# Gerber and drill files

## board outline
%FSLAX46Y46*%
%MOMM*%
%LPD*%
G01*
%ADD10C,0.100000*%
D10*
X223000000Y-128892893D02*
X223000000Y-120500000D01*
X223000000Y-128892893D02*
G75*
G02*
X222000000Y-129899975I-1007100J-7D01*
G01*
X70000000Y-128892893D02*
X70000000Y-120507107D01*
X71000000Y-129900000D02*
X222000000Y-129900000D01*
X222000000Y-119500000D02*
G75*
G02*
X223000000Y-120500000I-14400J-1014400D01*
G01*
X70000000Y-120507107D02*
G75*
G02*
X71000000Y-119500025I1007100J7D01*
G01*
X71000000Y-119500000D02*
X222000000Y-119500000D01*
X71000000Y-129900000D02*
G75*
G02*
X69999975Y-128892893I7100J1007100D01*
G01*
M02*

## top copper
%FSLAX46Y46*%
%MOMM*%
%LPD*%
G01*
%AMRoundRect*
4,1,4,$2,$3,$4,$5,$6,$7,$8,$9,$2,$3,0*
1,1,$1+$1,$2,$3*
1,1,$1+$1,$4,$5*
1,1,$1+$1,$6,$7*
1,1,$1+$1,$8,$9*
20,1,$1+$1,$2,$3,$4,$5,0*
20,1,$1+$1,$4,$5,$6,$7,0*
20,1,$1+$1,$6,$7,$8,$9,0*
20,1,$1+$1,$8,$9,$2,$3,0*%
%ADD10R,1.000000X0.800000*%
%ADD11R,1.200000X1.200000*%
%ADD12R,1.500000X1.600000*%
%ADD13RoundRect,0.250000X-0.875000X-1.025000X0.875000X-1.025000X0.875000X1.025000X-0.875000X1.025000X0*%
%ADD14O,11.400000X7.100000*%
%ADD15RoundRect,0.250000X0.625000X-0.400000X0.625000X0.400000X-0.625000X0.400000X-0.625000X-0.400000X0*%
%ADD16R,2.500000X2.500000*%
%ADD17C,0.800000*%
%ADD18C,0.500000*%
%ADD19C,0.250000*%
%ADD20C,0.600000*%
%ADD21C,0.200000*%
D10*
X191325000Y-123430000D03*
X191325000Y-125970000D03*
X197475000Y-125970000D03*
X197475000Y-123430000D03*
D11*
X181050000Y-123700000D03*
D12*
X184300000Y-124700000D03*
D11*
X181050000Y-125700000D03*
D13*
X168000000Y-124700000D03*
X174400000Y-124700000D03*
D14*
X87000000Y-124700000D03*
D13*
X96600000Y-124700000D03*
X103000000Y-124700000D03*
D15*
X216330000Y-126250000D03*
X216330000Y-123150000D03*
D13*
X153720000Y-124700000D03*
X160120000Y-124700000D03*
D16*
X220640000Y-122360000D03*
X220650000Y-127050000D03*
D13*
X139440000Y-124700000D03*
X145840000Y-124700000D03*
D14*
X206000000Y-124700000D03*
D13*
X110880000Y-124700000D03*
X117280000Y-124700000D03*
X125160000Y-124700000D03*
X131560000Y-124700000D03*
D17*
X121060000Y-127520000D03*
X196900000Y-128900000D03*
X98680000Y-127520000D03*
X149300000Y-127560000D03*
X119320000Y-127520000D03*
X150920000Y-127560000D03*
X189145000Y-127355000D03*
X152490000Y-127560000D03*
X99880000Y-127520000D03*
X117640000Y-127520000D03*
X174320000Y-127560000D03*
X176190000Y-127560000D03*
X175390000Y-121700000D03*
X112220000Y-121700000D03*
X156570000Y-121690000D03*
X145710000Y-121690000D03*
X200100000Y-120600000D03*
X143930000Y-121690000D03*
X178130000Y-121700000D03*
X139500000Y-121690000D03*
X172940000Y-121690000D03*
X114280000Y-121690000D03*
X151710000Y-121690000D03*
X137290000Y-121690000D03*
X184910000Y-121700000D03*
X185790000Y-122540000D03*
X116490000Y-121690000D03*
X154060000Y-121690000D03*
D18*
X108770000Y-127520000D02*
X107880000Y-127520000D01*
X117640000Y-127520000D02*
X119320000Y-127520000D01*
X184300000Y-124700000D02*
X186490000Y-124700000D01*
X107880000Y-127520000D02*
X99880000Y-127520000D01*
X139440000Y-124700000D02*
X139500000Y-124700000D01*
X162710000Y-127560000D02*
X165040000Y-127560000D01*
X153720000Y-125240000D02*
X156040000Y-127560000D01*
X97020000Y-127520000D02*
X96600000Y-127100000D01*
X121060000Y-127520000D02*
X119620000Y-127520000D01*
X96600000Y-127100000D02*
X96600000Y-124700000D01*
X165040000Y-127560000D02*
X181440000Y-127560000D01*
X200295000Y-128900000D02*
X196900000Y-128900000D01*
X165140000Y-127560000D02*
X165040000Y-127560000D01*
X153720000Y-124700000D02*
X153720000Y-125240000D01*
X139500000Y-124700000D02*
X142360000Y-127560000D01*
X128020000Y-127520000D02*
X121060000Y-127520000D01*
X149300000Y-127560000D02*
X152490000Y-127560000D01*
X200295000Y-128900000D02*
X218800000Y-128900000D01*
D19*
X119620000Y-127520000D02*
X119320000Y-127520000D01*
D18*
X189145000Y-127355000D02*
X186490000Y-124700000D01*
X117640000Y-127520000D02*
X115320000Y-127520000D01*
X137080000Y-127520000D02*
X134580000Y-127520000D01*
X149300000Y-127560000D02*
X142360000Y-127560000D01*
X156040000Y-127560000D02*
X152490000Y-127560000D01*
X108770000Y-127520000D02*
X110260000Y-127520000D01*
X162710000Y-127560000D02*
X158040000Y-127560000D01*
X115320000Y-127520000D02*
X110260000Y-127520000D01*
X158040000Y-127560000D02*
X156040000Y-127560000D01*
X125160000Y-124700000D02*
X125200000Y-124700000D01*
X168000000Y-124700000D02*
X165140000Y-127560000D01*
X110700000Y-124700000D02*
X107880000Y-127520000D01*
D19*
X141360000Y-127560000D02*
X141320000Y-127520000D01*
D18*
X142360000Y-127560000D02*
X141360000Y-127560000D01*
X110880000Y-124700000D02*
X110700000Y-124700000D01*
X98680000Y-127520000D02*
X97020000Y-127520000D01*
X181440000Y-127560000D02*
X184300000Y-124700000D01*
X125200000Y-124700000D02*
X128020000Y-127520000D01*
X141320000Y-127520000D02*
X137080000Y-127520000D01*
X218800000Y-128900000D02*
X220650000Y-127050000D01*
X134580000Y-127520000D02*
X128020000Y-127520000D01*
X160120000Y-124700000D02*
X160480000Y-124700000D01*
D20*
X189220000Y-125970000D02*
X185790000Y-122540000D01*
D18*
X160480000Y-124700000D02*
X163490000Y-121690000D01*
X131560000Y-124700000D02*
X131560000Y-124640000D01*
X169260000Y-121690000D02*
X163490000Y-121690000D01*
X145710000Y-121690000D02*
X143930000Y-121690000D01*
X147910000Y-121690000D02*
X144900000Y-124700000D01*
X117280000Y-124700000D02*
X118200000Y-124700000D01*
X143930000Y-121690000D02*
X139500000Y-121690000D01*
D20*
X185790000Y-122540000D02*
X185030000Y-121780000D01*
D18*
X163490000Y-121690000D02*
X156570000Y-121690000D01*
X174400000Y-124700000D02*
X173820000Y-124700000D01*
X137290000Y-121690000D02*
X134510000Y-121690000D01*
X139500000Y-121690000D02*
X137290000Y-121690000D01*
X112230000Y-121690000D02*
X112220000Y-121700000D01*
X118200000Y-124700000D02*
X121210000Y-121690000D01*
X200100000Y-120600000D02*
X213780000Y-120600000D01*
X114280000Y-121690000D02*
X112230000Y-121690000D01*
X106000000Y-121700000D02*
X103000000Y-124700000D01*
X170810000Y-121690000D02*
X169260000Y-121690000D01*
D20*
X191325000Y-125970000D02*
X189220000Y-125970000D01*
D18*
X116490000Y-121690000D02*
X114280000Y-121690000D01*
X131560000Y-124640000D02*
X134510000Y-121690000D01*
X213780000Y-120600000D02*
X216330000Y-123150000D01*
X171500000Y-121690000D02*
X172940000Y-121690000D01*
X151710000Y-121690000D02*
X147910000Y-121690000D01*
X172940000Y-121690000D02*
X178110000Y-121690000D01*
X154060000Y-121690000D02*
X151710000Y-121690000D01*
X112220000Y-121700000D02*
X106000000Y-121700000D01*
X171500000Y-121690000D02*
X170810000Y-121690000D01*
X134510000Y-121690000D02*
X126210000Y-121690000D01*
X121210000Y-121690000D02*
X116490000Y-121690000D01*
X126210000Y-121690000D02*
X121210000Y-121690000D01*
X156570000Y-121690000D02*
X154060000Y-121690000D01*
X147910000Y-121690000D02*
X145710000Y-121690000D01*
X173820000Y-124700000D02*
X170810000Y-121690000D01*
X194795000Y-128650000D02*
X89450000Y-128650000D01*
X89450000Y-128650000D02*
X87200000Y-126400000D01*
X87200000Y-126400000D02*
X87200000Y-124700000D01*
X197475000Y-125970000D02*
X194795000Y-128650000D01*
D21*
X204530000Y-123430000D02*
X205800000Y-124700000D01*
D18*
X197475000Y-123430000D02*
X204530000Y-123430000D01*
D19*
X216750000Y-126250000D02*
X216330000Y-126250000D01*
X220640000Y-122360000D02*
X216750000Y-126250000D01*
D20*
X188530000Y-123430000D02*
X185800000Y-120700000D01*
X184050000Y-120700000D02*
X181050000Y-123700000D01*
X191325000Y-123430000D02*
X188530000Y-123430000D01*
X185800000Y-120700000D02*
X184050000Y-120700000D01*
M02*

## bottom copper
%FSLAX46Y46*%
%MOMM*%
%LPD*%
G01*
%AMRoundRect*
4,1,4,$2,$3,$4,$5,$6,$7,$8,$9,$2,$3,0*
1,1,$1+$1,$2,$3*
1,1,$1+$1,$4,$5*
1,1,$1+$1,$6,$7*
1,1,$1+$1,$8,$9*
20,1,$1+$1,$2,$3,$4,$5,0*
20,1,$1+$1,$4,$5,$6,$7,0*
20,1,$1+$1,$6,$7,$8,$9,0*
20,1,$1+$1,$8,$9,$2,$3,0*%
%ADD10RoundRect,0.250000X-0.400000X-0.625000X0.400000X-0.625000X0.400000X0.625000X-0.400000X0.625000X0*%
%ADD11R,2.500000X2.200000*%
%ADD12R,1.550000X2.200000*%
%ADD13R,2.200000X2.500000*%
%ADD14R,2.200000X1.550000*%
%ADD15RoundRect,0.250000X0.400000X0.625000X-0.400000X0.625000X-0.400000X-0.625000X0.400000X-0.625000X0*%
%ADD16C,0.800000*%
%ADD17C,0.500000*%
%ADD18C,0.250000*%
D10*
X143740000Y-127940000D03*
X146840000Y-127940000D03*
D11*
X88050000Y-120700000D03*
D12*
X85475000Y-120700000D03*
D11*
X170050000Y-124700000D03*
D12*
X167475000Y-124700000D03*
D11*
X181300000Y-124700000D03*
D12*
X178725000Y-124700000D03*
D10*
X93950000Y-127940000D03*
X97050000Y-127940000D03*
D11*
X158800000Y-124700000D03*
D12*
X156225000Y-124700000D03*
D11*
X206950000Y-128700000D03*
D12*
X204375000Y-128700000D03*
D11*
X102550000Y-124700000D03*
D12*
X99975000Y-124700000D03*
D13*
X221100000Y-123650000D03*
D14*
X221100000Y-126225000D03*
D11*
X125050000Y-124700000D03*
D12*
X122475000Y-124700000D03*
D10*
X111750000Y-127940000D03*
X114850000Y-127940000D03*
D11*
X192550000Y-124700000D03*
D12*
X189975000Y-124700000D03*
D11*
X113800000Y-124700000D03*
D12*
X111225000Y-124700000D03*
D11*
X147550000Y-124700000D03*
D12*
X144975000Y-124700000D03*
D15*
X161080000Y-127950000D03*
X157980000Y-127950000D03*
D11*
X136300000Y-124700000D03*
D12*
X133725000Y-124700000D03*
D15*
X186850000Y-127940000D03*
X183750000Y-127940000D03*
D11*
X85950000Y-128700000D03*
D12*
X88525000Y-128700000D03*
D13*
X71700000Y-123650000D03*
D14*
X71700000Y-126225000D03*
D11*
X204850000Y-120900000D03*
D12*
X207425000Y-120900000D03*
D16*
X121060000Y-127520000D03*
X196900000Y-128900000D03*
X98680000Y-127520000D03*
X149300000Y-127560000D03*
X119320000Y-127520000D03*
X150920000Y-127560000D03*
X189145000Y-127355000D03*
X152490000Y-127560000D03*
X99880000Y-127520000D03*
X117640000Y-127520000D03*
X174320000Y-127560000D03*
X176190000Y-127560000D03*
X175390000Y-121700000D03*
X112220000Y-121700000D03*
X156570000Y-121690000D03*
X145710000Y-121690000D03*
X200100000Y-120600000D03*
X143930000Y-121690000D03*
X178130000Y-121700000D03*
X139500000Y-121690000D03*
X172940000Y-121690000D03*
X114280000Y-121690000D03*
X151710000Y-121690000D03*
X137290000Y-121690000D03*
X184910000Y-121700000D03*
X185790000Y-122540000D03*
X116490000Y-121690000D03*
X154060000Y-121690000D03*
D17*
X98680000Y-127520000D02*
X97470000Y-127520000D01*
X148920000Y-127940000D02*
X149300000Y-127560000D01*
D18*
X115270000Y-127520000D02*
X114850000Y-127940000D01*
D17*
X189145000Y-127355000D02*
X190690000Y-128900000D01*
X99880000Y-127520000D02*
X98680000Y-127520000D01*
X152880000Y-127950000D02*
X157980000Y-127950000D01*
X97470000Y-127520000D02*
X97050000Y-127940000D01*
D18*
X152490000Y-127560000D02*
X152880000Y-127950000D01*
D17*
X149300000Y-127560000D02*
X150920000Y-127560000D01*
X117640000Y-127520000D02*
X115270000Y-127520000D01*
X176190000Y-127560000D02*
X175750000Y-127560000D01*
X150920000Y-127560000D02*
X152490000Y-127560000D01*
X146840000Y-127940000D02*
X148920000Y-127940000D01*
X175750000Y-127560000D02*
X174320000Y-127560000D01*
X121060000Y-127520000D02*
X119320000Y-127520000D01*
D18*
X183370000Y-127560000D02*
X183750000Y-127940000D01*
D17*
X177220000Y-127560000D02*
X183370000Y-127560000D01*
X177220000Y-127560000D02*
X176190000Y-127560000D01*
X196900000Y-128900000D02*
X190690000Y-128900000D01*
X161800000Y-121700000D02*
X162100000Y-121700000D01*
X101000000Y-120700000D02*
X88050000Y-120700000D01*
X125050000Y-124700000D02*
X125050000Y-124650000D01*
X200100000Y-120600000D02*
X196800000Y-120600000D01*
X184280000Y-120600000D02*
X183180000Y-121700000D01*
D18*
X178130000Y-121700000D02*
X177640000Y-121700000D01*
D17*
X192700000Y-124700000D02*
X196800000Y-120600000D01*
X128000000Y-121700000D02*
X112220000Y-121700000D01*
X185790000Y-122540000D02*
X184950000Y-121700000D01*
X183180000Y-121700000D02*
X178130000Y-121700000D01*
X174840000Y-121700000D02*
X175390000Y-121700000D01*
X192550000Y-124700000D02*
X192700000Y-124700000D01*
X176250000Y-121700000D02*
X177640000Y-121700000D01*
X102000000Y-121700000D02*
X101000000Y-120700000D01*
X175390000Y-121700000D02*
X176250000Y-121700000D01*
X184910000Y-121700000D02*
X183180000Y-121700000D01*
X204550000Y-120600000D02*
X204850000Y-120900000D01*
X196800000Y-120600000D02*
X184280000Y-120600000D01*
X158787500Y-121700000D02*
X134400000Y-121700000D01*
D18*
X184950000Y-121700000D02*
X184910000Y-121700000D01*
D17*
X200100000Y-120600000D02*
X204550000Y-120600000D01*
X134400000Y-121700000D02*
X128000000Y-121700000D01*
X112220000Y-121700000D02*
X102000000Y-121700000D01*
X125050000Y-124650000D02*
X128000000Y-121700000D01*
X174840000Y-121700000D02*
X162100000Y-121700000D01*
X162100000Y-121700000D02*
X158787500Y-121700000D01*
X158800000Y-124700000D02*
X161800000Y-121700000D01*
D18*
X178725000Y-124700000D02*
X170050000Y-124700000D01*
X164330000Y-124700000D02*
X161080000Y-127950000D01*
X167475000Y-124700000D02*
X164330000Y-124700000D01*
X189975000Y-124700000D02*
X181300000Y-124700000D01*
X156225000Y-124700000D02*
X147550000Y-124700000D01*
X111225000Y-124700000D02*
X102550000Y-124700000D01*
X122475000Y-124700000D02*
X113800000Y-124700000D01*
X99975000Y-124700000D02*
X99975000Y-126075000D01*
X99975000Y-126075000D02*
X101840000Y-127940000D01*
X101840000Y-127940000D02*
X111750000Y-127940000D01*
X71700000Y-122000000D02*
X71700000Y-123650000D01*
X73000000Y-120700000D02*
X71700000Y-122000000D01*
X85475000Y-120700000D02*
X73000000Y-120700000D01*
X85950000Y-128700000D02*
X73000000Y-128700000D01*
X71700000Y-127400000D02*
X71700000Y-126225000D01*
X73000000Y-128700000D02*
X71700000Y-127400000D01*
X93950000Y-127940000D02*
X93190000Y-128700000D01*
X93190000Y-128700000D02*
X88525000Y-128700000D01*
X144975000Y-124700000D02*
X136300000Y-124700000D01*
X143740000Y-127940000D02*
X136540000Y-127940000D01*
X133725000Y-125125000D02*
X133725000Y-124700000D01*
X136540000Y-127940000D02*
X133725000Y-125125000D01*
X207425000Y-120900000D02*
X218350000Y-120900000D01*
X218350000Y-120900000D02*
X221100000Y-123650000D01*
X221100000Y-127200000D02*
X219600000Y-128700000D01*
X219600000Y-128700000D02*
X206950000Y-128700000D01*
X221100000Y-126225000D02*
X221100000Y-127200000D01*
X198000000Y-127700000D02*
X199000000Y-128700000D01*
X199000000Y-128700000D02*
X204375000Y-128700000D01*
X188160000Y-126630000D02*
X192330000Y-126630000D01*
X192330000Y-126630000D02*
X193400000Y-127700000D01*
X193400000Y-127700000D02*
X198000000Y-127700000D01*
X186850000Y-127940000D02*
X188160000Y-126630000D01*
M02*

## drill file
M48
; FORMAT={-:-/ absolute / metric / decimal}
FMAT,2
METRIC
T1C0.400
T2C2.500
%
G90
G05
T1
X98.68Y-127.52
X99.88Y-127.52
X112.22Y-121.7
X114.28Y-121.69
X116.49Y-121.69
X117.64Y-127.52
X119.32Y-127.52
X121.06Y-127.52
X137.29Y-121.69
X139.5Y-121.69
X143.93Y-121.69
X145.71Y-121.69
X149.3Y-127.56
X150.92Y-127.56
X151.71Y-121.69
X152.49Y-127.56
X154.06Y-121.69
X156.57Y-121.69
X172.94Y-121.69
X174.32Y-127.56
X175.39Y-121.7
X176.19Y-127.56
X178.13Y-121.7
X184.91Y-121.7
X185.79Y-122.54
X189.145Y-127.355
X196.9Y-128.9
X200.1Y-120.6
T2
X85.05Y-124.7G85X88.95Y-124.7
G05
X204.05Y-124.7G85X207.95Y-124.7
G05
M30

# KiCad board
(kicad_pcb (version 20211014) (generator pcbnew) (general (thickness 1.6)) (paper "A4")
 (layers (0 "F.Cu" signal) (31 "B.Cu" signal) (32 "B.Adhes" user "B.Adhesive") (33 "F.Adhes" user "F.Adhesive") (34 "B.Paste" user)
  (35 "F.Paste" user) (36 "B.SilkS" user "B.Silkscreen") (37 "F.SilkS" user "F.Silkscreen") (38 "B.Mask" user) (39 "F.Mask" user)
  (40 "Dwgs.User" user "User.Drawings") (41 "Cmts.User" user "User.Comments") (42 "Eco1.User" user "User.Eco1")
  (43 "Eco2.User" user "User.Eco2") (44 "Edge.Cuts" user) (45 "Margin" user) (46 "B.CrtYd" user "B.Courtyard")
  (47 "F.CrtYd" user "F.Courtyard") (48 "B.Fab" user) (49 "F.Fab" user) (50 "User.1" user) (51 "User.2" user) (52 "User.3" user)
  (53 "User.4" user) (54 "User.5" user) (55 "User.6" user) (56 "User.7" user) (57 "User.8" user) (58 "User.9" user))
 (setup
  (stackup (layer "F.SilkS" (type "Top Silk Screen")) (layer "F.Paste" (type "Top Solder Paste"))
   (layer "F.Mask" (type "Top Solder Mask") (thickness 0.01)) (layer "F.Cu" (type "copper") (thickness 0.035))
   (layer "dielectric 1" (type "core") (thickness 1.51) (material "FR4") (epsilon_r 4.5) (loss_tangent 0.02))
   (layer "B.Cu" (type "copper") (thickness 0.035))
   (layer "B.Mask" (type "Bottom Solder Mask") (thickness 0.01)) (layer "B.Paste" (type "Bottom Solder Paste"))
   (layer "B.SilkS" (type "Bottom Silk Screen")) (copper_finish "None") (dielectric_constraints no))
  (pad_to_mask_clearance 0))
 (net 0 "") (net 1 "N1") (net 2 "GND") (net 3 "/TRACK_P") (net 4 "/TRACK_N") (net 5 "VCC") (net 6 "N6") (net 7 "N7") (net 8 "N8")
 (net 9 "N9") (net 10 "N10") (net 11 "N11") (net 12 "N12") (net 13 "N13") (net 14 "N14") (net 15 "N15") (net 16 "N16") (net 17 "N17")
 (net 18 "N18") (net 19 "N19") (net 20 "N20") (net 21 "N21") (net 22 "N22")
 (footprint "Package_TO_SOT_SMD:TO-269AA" (layer "F.Cu") (at 194.4 124.7)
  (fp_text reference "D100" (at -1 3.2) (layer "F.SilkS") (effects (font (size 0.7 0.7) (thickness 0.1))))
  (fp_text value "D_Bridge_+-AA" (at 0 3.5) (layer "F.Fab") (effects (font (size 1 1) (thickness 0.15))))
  (pad "1" smd rect (at -3.075 -1.27) (size 1 0.8) (layers "F.Cu" "F.Paste" "F.Mask") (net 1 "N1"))
  (pad "2" smd rect (at -3.075 1.27) (size 1 0.8) (layers "F.Cu" "F.Paste" "F.Mask") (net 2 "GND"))
  (pad "3" smd rect (at 3.075 1.27) (size 1 0.8) (layers "F.Cu" "F.Paste" "F.Mask") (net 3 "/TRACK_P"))
  (pad "4" smd rect (at 3.075 -1.27) (size 1 0.8) (layers "F.Cu" "F.Paste" "F.Mask") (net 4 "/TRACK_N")))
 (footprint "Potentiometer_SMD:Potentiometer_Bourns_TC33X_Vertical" (layer "F.Cu") (at 182.85 124.7)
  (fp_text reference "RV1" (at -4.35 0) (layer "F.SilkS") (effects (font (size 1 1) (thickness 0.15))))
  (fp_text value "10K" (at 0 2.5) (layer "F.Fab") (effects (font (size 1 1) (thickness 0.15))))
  (pad "1" smd rect (at -1.8 -1) (size 1.2 1.2) (layers "F.Cu" "F.Paste" "F.Mask") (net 1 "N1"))
  (pad "2" smd rect (at 1.45 0) (size 1.5 1.6) (layers "F.Cu" "F.Paste" "F.Mask") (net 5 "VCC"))
  (pad "3" smd rect (at -1.8 1) (size 1.2 1.2) (layers "F.Cu" "F.Paste" "F.Mask") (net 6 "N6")))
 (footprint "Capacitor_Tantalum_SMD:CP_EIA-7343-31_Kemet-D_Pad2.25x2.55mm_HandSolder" (layer "F.Cu") (at 171.2 124.7)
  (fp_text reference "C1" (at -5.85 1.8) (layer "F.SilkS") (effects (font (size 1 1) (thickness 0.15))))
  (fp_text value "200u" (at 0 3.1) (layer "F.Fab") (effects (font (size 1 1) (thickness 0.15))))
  (pad "1" smd roundrect (at -3.2 0) (size 2.25 2.55) (layers "F.Cu" "F.Paste" "F.Mask") (roundrect_rratio 0.1111111111) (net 5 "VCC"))
  (pad "2" smd roundrect (at 3.2 0) (size 2.25 2.55) (layers "F.Cu" "F.Paste" "F.Mask") (roundrect_rratio 0.1111111111) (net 2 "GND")))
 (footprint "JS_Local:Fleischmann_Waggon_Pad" (layer "F.Cu") (at 85.5 124.7)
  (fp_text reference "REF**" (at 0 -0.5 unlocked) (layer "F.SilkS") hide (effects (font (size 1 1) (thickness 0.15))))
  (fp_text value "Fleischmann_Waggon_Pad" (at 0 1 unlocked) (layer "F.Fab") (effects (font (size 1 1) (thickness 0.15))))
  (pad "1" thru_hole oval (at 1.5 0) (size 11.4 7.1) (drill oval 6.4 2.5) (layers *.Cu "F.Mask") (remove_unused_layers) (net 3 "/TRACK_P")))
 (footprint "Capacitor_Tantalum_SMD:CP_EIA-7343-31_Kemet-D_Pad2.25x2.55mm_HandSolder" (layer "F.Cu") (at 99.8 124.7)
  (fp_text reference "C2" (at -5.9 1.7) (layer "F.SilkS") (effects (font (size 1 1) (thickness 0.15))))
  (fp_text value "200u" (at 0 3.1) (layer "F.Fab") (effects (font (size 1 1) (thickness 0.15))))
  (pad "1" smd roundrect (at -3.2 0) (size 2.25 2.55) (layers "F.Cu" "F.Paste" "F.Mask") (roundrect_rratio 0.1111111111) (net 5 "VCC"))
  (pad "2" smd roundrect (at 3.2 0) (size 2.25 2.55) (layers "F.Cu" "F.Paste" "F.Mask") (roundrect_rratio 0.1111111111) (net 2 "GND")))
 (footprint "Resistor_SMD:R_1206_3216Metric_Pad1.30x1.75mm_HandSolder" (layer "F.Cu") (at 216.33 124.7 90)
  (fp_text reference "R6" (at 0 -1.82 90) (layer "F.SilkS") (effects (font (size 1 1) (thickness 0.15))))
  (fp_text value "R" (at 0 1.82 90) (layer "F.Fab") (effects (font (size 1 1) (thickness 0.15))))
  (pad "1" smd roundrect (at -1.55 0 90) (size 1.3 1.75) (layers "F.Cu" "F.Paste" "F.Mask") (roundrect_rratio 0.1923076923) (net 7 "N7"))
  (pad "2" smd roundrect (at 1.55 0 90) (size 1.3 1.75) (layers "F.Cu" "F.Paste" "F.Mask") (roundrect_rratio 0.1923076923) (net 2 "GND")))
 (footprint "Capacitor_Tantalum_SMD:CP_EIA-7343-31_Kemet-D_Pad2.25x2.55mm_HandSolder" (layer "F.Cu") (at 156.92 124.7)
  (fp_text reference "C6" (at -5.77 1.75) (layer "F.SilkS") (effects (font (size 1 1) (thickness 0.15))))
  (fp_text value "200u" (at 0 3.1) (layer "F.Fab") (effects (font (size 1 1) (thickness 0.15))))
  (pad "1" smd roundrect (at -3.2 0) (size 2.25 2.55) (layers "F.Cu" "F.Paste" "F.Mask") (roundrect_rratio 0.111111) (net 5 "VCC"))
  (pad "2" smd roundrect (at 3.2 0) (size 2.25 2.55) (layers "F.Cu" "F.Paste" "F.Mask") (roundrect_rratio 0.111111) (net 2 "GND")))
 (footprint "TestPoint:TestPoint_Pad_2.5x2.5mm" (layer "F.Cu") (at 220.64 122.36)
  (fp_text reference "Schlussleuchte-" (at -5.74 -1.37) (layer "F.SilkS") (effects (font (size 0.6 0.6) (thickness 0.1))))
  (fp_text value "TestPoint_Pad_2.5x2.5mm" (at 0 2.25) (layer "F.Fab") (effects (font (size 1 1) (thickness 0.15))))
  (pad "1" smd rect (at 0 0) (size 2.5 2.5) (layers "F.Cu" "F.Mask") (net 7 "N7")))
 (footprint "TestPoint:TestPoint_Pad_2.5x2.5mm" (layer "F.Cu") (at 220.65 127.05)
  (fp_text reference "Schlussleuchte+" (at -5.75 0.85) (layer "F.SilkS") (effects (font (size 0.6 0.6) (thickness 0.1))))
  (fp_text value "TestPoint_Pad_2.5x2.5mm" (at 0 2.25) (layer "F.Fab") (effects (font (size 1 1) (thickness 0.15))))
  (pad "1" smd rect (at 0 0) (size 2.5 2.5) (layers "F.Cu" "F.Mask") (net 5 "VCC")))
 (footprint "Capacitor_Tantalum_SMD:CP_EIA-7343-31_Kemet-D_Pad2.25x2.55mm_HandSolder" (layer "F.Cu") (at 142.64 124.7)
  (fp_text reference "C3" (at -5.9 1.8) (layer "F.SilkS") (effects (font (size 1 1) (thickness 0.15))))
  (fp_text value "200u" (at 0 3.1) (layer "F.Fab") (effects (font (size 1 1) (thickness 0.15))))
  (pad "1" smd roundrect (at -3.2 0) (size 2.25 2.55) (layers "F.Cu" "F.Paste" "F.Mask") (roundrect_rratio 0.1111111111) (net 5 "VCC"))
  (pad "2" smd roundrect (at 3.2 0) (size 2.25 2.55) (layers "F.Cu" "F.Paste" "F.Mask") (roundrect_rratio 0.1111111111) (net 2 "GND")))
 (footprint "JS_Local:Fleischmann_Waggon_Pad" (layer "F.Cu") (at 207.7 124.7)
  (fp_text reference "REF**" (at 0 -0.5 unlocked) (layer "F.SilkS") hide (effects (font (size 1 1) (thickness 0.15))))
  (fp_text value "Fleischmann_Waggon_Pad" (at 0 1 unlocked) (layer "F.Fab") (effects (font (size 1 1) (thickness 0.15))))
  (pad "1" thru_hole oval (at -1.7 0) (size 11.4 7.1) (drill oval 6.4 2.5) (layers *.Cu "F.Mask") (remove_unused_layers) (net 4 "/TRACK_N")))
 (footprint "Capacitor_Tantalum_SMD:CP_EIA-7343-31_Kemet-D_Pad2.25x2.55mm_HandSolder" (layer "F.Cu") (at 114.08 124.7)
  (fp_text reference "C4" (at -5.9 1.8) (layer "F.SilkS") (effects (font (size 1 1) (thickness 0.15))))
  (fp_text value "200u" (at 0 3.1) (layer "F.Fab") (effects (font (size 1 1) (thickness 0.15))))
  (pad "1" smd roundrect (at -3.2 0) (size 2.25 2.55) (layers "F.Cu" "F.Paste" "F.Mask") (roundrect_rratio 0.1111111111) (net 5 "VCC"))
  (pad "2" smd roundrect (at 3.2 0) (size 2.25 2.55) (layers "F.Cu" "F.Paste" "F.Mask") (roundrect_rratio 0.1111111111) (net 2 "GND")))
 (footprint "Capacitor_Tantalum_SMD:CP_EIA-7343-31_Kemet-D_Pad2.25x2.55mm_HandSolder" (layer "F.Cu") (at 128.36 124.7)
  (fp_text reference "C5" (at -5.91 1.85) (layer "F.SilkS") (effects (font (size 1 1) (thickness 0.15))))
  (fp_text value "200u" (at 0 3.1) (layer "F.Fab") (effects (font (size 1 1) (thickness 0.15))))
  (pad "1" smd roundrect (at -3.2 0) (size 2.25 2.55) (layers "F.Cu" "F.Paste" "F.Mask") (roundrect_rratio 0.111111) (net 5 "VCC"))
  (pad "2" smd roundrect (at 3.2 0) (size 2.25 2.55) (layers "F.Cu" "F.Paste" "F.Mask") (roundrect_rratio 0.111111) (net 2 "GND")))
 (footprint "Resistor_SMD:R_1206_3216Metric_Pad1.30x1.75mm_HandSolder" (layer "B.Cu") (at 145.29 127.94)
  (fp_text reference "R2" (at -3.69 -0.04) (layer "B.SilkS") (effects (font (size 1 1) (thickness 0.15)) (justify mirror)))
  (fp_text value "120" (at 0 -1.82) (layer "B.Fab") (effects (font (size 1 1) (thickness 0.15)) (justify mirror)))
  (pad "1" smd roundrect (at -1.55 0) (size 1.3 1.75) (layers "B.Cu" "B.Paste" "B.Mask") (roundrect_rratio 0.1923076923) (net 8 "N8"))
  (pad "2" smd roundrect (at 1.55 0) (size 1.3 1.75) (layers "B.Cu" "B.Paste" "B.Mask") (roundrect_rratio 0.1923076923) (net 5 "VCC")))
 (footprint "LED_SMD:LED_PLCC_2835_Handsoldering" (layer "B.Cu") (at 87 120.7 180)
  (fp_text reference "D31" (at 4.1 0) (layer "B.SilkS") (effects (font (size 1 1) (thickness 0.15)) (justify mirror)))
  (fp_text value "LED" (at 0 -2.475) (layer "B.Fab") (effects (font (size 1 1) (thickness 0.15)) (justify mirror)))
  (pad "1" smd rect (at -1.05 0 180) (size 2.5 2.2) (layers "B.Cu" "B.Paste" "B.Mask") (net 2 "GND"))
  (pad "2" smd rect (at 1.525 0 180) (size 1.55 2.2) (layers "B.Cu" "B.Paste" "B.Mask") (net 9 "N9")))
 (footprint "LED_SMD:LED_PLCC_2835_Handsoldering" (layer "B.Cu") (at 169 124.7 180)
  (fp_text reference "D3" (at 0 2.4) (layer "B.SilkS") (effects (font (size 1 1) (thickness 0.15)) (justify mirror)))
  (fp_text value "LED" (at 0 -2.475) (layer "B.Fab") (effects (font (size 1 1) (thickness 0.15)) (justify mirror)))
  (pad "1" smd rect (at -1.05 0 180) (size 2.5 2.2) (layers "B.Cu" "B.Paste" "B.Mask") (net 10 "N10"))
  (pad "2" smd rect (at 1.525 0 180) (size 1.55 2.2) (layers "B.Cu" "B.Paste" "B.Mask") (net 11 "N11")))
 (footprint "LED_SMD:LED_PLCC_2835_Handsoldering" (layer "B.Cu") (at 180.25 124.7 180)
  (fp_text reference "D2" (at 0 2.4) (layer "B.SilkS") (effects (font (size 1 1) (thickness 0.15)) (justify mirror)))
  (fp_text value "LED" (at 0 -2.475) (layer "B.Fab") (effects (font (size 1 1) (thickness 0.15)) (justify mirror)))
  (pad "1" smd rect (at -1.05 0 180) (size 2.5 2.2) (layers "B.Cu" "B.Paste" "B.Mask") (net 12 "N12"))
  (pad "2" smd rect (at 1.525 0 180) (size 1.55 2.2) (layers "B.Cu" "B.Paste" "B.Mask") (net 10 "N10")))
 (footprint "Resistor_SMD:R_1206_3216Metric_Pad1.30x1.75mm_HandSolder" (layer "B.Cu") (at 95.5 127.94)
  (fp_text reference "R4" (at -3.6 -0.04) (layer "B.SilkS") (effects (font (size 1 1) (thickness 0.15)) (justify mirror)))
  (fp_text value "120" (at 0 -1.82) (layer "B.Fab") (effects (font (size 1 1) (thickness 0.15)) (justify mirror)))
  (pad "1" smd roundrect (at -1.55 0) (size 1.3 1.75) (layers "B.Cu" "B.Paste" "B.Mask") (roundrect_rratio 0.1923076923) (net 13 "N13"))
  (pad "2" smd roundrect (at 1.55 0) (size 1.3 1.75) (layers "B.Cu" "B.Paste" "B.Mask") (roundrect_rratio 0.1923076923) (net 5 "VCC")))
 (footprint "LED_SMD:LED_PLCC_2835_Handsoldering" (layer "B.Cu") (at 157.75 124.7 180)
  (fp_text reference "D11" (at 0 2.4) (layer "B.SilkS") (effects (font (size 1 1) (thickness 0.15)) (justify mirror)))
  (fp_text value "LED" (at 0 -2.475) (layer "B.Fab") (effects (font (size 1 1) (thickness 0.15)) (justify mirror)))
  (pad "1" smd rect (at -1.05 0 180) (size 2.5 2.2) (layers "B.Cu" "B.Paste" "B.Mask") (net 2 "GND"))
  (pad "2" smd rect (at 1.525 0 180) (size 1.55 2.2) (layers "B.Cu" "B.Paste" "B.Mask") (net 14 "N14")))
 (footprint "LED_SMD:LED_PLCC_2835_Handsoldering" (layer "B.Cu") (at 205.9 128.7 180)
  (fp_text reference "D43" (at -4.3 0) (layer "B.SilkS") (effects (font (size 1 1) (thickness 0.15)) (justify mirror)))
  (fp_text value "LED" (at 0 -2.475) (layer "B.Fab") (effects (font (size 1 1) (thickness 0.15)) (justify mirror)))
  (pad "1" smd rect (at -1.05 0 180) (size 2.5 2.2) (layers "B.Cu" "B.Paste" "B.Mask") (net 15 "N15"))
  (pad "2" smd rect (at 1.525 0 180) (size 1.55 2.2) (layers "B.Cu" "B.Paste" "B.Mask") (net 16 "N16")))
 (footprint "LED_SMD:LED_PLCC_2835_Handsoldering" (layer "B.Cu") (at 101.5 124.7 180)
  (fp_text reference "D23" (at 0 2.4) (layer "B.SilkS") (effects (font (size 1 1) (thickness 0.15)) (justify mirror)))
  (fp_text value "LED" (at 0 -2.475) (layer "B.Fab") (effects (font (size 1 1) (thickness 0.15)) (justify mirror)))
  (pad "1" smd rect (at -1.05 0 180) (size 2.5 2.2) (layers "B.Cu" "B.Paste" "B.Mask") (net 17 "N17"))
  (pad "2" smd rect (at 1.525 0 180) (size 1.55 2.2) (layers "B.Cu" "B.Paste" "B.Mask") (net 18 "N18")))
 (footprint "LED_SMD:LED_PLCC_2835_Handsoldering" (layer "B.Cu") (at 221.1 124.7 -90)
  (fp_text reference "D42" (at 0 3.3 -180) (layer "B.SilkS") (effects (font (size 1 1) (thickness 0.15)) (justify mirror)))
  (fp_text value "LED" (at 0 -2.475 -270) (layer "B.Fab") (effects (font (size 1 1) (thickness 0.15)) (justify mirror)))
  (pad "1" smd rect (at -1.05 0 270) (size 2.5 2.2) (layers "B.Cu" "B.Paste" "B.Mask") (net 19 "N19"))
  (pad "2" smd rect (at 1.525 0 270) (size 1.55 2.2) (layers "B.Cu" "B.Paste" "B.Mask") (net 15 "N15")))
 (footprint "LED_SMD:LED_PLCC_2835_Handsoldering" (layer "B.Cu") (at 124 124.7 180)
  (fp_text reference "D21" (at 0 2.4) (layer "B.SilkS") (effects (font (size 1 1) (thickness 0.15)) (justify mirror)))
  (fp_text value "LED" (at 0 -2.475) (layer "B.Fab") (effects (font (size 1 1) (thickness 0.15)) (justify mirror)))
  (pad "1" smd rect (at -1.05 0 180) (size 2.5 2.2) (layers "B.Cu" "B.Paste" "B.Mask") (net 2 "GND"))
  (pad "2" smd rect (at 1.525 0 180) (size 1.55 2.2) (layers "B.Cu" "B.Paste" "B.Mask") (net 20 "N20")))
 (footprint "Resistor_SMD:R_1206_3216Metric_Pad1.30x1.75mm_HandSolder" (layer "B.Cu") (at 113.3 127.94)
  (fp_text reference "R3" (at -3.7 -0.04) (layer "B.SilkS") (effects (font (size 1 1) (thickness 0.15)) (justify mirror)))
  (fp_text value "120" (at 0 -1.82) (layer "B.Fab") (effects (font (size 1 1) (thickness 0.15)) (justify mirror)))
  (pad "1" smd roundrect (at -1.55 0) (size 1.3 1.75) (layers "B.Cu" "B.Paste" "B.Mask") (roundrect_rratio 0.1923076923) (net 18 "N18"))
  (pad "2" smd roundrect (at 1.55 0) (size 1.3 1.75) (layers "B.Cu" "B.Paste" "B.Mask") (roundrect_rratio 0.1923076923) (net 5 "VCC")))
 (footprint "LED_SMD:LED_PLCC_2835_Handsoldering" (layer "B.Cu") (at 191.5 124.7 180)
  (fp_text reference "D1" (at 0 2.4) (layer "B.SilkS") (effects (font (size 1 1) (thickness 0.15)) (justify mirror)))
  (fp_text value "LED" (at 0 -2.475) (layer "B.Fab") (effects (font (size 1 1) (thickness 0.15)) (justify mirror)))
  (pad "1" smd rect (at -1.05 0 180) (size 2.5 2.2) (layers "B.Cu" "B.Paste" "B.Mask") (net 2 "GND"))
  (pad "2" smd rect (at 1.525 0 180) (size 1.55 2.2) (layers "B.Cu" "B.Paste" "B.Mask") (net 12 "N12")))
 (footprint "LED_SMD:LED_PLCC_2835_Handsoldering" (layer "B.Cu") (at 112.75 124.7 180)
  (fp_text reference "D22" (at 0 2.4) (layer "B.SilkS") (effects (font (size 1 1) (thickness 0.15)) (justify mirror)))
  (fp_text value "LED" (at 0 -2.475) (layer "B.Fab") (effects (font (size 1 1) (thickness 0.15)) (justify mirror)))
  (pad "1" smd rect (at -1.05 0 180) (size 2.5 2.2) (layers "B.Cu" "B.Paste" "B.Mask") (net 20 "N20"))
  (pad "2" smd rect (at 1.525 0 180) (size 1.55 2.2) (layers "B.Cu" "B.Paste" "B.Mask") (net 17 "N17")))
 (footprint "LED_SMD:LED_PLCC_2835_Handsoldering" (layer "B.Cu") (at 146.5 124.7 180)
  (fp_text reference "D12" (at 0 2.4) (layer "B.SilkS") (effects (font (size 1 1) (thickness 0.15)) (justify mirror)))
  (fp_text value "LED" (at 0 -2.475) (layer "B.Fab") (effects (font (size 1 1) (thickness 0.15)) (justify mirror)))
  (pad "1" smd rect (at -1.05 0 180) (size 2.5 2.2) (layers "B.Cu" "B.Paste" "B.Mask") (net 14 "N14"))
  (pad "2" smd rect (at 1.525 0 180) (size 1.55 2.2) (layers "B.Cu" "B.Paste" "B.Mask") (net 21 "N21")))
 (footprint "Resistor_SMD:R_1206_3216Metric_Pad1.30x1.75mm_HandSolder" (layer "B.Cu") (at 159.53 127.95 180)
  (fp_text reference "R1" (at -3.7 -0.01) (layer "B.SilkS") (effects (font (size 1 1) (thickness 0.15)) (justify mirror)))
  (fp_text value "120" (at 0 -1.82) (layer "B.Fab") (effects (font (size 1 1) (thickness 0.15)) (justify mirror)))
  (pad "1" smd roundrect (at -1.55 0 180) (size 1.3 1.75) (layers "B.Cu" "B.Paste" "B.Mask") (roundrect_rratio 0.1923076923) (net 11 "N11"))
  (pad "2" smd roundrect (at 1.55 0 180) (size 1.3 1.75) (layers "B.Cu" "B.Paste" "B.Mask") (roundrect_rratio 0.1923076923) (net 5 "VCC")))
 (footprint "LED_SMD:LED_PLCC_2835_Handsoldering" (layer "B.Cu") (at 135.25 124.7 180)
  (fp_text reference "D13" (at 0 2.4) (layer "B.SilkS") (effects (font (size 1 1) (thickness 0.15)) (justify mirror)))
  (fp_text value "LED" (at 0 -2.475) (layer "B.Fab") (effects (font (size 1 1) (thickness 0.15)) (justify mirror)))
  (pad "1" smd rect (at -1.05 0 180) (size 2.5 2.2) (layers "B.Cu" "B.Paste" "B.Mask") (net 21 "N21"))
  (pad "2" smd rect (at 1.525 0 180) (size 1.55 2.2) (layers "B.Cu" "B.Paste" "B.Mask") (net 8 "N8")))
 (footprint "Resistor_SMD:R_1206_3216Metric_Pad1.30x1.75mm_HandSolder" (layer "B.Cu") (at 185.3 127.94 180)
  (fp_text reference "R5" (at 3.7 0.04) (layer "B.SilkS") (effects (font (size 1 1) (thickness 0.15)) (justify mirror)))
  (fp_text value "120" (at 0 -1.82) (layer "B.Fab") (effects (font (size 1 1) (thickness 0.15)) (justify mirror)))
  (pad "1" smd roundrect (at -1.55 0 180) (size 1.3 1.75) (layers "B.Cu" "B.Paste" "B.Mask") (roundrect_rratio 0.1923076923) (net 16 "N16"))
  (pad "2" smd roundrect (at 1.55 0 180) (size 1.3 1.75) (layers "B.Cu" "B.Paste" "B.Mask") (roundrect_rratio 0.1923076923) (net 5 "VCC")))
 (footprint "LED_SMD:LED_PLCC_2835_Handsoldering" (layer "B.Cu") (at 87 128.7)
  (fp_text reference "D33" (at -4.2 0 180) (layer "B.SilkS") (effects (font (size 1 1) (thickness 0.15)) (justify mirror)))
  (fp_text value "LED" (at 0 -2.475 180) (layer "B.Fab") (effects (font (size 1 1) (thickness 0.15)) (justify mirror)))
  (pad "1" smd rect (at -1.05 0) (size 2.5 2.2) (layers "B.Cu" "B.Paste" "B.Mask") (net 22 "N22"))
  (pad "2" smd rect (at 1.525 0) (size 1.55 2.2) (layers "B.Cu" "B.Paste" "B.Mask") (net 13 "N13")))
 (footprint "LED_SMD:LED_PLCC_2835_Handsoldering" (layer "B.Cu") (at 71.7 124.7 -90)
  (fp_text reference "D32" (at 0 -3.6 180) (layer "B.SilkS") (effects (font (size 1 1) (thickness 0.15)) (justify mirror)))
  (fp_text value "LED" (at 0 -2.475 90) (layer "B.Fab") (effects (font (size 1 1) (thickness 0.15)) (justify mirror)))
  (pad "1" smd rect (at -1.05 0 270) (size 2.5 2.2) (layers "B.Cu" "B.Paste" "B.Mask") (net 9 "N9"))
  (pad "2" smd rect (at 1.525 0 270) (size 1.55 2.2) (layers "B.Cu" "B.Paste" "B.Mask") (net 22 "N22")))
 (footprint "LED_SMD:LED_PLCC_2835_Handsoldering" (layer "B.Cu") (at 205.9 120.9)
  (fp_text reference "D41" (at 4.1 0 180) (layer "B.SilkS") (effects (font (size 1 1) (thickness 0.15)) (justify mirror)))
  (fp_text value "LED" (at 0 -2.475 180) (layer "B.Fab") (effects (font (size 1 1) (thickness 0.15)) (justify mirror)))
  (pad "1" smd rect (at -1.05 0) (size 2.5 2.2) (layers "B.Cu" "B.Paste" "B.Mask") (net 2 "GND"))
  (pad "2" smd rect (at 1.525 0) (size 1.55 2.2) (layers "B.Cu" "B.Paste" "B.Mask") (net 19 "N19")))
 (gr_line (start 223 128.892893) (end 223 120.5) (layer "Edge.Cuts") (width 0.1))
 (gr_arc (start 223 128.892893) (mid 222.707535 129.602517) (end 222 129.9) (layer "Edge.Cuts") (width 0.1))
 (gr_line (start 70 128.892893) (end 70 120.507107) (layer "Edge.Cuts") (width 0.1))
 (gr_line (start 71 129.9) (end 222 129.9) (layer "Edge.Cuts") (width 0.1))
 (gr_arc (start 222 119.5) (mid 222.702951 119.797049) (end 223 120.5) (layer "Edge.Cuts") (width 0.1))
 (gr_arc (start 70 120.507107) (mid 70.292465 119.797483) (end 71 119.5) (layer "Edge.Cuts") (width 0.1))
 (gr_line (start 71 119.5) (end 222 119.5) (layer "Edge.Cuts") (width 0.1))
 (gr_arc (start 71 129.9) (mid 70.292465 129.602517) (end 70 128.892893) (layer "Edge.Cuts") (width 0.1))
 (segment (start 108.77 127.52) (end 107.88 127.52) (width 0.5) (layer "F.Cu") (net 5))
 (segment (start 117.64 127.52) (end 119.32 127.52) (width 0.5) (layer "F.Cu") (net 5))
 (segment (start 184.3 124.7) (end 186.49 124.7) (width 0.5) (layer "F.Cu") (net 5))
 (segment (start 107.88 127.52) (end 99.88 127.52) (width 0.5) (layer "F.Cu") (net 5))
 (segment (start 139.44 124.7) (end 139.5 124.7) (width 0.5) (layer "F.Cu") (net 5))
 (segment (start 162.71 127.56) (end 165.04 127.56) (width 0.5) (layer "F.Cu") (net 5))
 (segment (start 153.72 125.24) (end 156.04 127.56) (width 0.5) (layer "F.Cu") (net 5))
 (segment (start 97.02 127.52) (end 96.6 127.1) (width 0.5) (layer "F.Cu") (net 5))
 (segment (start 121.06 127.52) (end 119.62 127.52) (width 0.5) (layer "F.Cu") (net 5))
 (segment (start 96.6 127.1) (end 96.6 124.7) (width 0.5) (layer "F.Cu") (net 5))
 (segment (start 165.04 127.56) (end 181.44 127.56) (width 0.5) (layer "F.Cu") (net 5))
 (segment (start 200.295 128.9) (end 196.9 128.9) (width 0.5) (layer "F.Cu") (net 5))
 (segment (start 165.14 127.56) (end 165.04 127.56) (width 0.5) (layer "F.Cu") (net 5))
 (segment (start 153.72 124.7) (end 153.72 125.24) (width 0.5) (layer "F.Cu") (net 5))
 (segment (start 139.5 124.7) (end 142.36 127.56) (width 0.5) (layer "F.Cu") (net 5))
 (segment (start 128.02 127.52) (end 121.06 127.52) (width 0.5) (layer "F.Cu") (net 5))
 (segment (start 149.3 127.56) (end 152.49 127.56) (width 0.5) (layer "F.Cu") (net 5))
 (segment (start 200.295 128.9) (end 218.8 128.9) (width 0.5) (layer "F.Cu") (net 5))
 (segment (start 119.62 127.52) (end 119.32 127.52) (width 0.25) (layer "F.Cu") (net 5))
 (segment (start 189.145 127.355) (end 186.49 124.7) (width 0.5) (layer "F.Cu") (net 5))
 (segment (start 117.64 127.52) (end 115.32 127.52) (width 0.5) (layer "F.Cu") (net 5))
 (segment (start 137.08 127.52) (end 134.58 127.52) (width 0.5) (layer "F.Cu") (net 5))
 (segment (start 149.3 127.56) (end 142.36 127.56) (width 0.5) (layer "F.Cu") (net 5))
 (segment (start 156.04 127.56) (end 152.49 127.56) (width 0.5) (layer "F.Cu") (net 5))
 (segment (start 108.77 127.52) (end 110.26 127.52) (width 0.5) (layer "F.Cu") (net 5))
 (segment (start 162.71 127.56) (end 158.04 127.56) (width 0.5) (layer "F.Cu") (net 5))
 (segment (start 115.32 127.52) (end 110.26 127.52) (width 0.5) (layer "F.Cu") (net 5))
 (segment (start 158.04 127.56) (end 156.04 127.56) (width 0.5) (layer "F.Cu") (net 5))
 (segment (start 125.16 124.7) (end 125.2 124.7) (width 0.5) (layer "F.Cu") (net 5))
 (segment (start 168 124.7) (end 165.14 127.56) (width 0.5) (layer "F.Cu") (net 5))
 (segment (start 110.7 124.7) (end 107.88 127.52) (width 0.5) (layer "F.Cu") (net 5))
 (segment (start 141.36 127.56) (end 141.32 127.52) (width 0.25) (layer "F.Cu") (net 5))
 (segment (start 142.36 127.56) (end 141.36 127.56) (width 0.5) (layer "F.Cu") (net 5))
 (segment (start 110.88 124.7) (end 110.7 124.7) (width 0.5) (layer "F.Cu") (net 5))
 (segment (start 98.68 127.52) (end 97.02 127.52) (width 0.5) (layer "F.Cu") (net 5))
 (segment (start 181.44 127.56) (end 184.3 124.7) (width 0.5) (layer "F.Cu") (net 5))
 (segment (start 125.2 124.7) (end 128.02 127.52) (width 0.5) (layer "F.Cu") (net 5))
 (segment (start 141.32 127.52) (end 137.08 127.52) (width 0.5) (layer "F.Cu") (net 5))
 (segment (start 218.8 128.9) (end 220.65 127.05) (width 0.5) (layer "F.Cu") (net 5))
 (segment (start 134.58 127.52) (end 128.02 127.52) (width 0.5) (layer "F.Cu") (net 5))
 (via (at 121.06 127.52) (size 0.8) (drill 0.4) (layers "F.Cu" "B.Cu") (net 5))
 (via (at 196.9 128.9) (size 0.8) (drill 0.4) (layers "F.Cu" "B.Cu") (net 5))
 (via (at 98.68 127.52) (size 0.8) (drill 0.4) (layers "F.Cu" "B.Cu") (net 5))
 (via (at 149.3 127.56) (size 0.8) (drill 0.4) (layers "F.Cu" "B.Cu") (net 5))
 (via (at 119.32 127.52) (size 0.8) (drill 0.4) (layers "F.Cu" "B.Cu") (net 5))
 (via (at 150.92 127.56) (size 0.8) (drill 0.4) (layers "F.Cu" "B.Cu") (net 5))
 (via (at 189.145 127.355) (size 0.8) (drill 0.4) (layers "F.Cu" "B.Cu") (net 5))
 (via (at 152.49 127.56) (size 0.8) (drill 0.4) (layers "F.Cu" "B.Cu") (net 5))
 (via (at 99.88 127.52) (size 0.8) (drill 0.4) (layers "F.Cu" "B.Cu") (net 5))
 (via (at 117.64 127.52) (size 0.8) (drill 0.4) (layers "F.Cu" "B.Cu") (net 5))
 (via (at 174.32 127.56) (size 0.8) (drill 0.4) (layers "F.Cu" "B.Cu") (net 5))
 (via (at 176.19 127.56) (size 0.8) (drill 0.4) (layers "F.Cu" "B.Cu") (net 5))
 (segment (start 98.68 127.52) (end 97.47 127.52) (width 0.5) (layer "B.Cu") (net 5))
 (segment (start 148.92 127.94) (end 149.3 127.56) (width 0.5) (layer "B.Cu") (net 5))
 (segment (start 115.27 127.52) (end 114.85 127.94) (width 0.25) (layer "B.Cu") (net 5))
 (segment (start 189.145 127.355) (end 190.69 128.9) (width 0.5) (layer "B.Cu") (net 5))
 (segment (start 99.88 127.52) (end 98.68 127.52) (width 0.5) (layer "B.Cu") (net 5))
 (segment (start 152.88 127.95) (end 157.98 127.95) (width 0.5) (layer "B.Cu") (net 5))
 (segment (start 97.47 127.52) (end 97.05 127.94) (width 0.5) (layer "B.Cu") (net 5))
 (segment (start 152.49 127.56) (end 152.88 127.95) (width 0.25) (layer "B.Cu") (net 5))
 (segment (start 149.3 127.56) (end 150.92 127.56) (width 0.5) (layer "B.Cu") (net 5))
 (segment (start 117.64 127.52) (end 115.27 127.52) (width 0.5) (layer "B.Cu") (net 5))
 (segment (start 176.19 127.56) (end 175.75 127.56) (width 0.5) (layer "B.Cu") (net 5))
 (segment (start 150.92 127.56) (end 152.49 127.56) (width 0.5) (layer "B.Cu") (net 5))
 (segment (start 146.84 127.94) (end 148.92 127.94) (width 0.5) (layer "B.Cu") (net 5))
 (segment (start 175.75 127.56) (end 174.32 127.56) (width 0.5) (layer "B.Cu") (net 5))
 (segment (start 121.06 127.52) (end 119.32 127.52) (width 0.5) (layer "B.Cu") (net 5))
 (segment (start 183.37 127.56) (end 183.75 127.94) (width 0.25) (layer "B.Cu") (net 5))
 (segment (start 177.22 127.56) (end 183.37 127.56) (width 0.5) (layer "B.Cu") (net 5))
 (segment (start 177.22 127.56) (end 176.19 127.56) (width 0.5) (layer "B.Cu") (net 5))
 (segment (start 196.9 128.9) (end 190.69 128.9) (width 0.5) (layer "B.Cu") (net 5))
 (segment (start 160.12 124.7) (end 160.48 124.7) (width 0.5) (layer "F.Cu") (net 2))
 (segment (start 189.22 125.97) (end 185.79 122.54) (width 0.6) (layer "F.Cu") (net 2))
 (segment (start 160.48 124.7) (end 163.49 121.69) (width 0.5) (layer "F.Cu") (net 2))
 (segment (start 131.56 124.7) (end 131.56 124.64) (width 0.5) (layer "F.Cu") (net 2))
 (segment (start 169.26 121.69) (end 163.49 121.69) (width 0.5) (layer "F.Cu") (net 2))
 (segment (start 145.71 121.69) (end 143.93 121.69) (width 0.5) (layer "F.Cu") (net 2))
 (segment (start 147.91 121.69) (end 144.9 124.7) (width 0.5) (layer "F.Cu") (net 2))
 (segment (start 117.28 124.7) (end 118.2 124.7) (width 0.5) (layer "F.Cu") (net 2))
 (segment (start 143.93 121.69) (end 139.5 121.69) (width 0.5) (layer "F.Cu") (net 2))
 (segment (start 185.79 122.54) (end 185.03 121.78) (width 0.6) (layer "F.Cu") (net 2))
 (segment (start 163.49 121.69) (end 156.57 121.69) (width 0.5) (layer "F.Cu") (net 2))
 (segment (start 174.4 124.7) (end 173.82 124.7) (width 0.5) (layer "F.Cu") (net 2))
 (segment (start 137.29 121.69) (end 134.51 121.69) (width 0.5) (layer "F.Cu") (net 2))
 (segment (start 139.5 121.69) (end 137.29 121.69) (width 0.5) (layer "F.Cu") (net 2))
 (segment (start 112.23 121.69) (end 112.22 121.7) (width 0.5) (layer "F.Cu") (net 2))
 (segment (start 118.2 124.7) (end 121.21 121.69) (width 0.5) (layer "F.Cu") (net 2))
 (segment (start 200.1 120.6) (end 213.78 120.6) (width 0.5) (layer "F.Cu") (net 2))
 (segment (start 114.28 121.69) (end 112.23 121.69) (width 0.5) (layer "F.Cu") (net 2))
 (segment (start 106 121.7) (end 103 124.7) (width 0.5) (layer "F.Cu") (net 2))
 (segment (start 170.81 121.69) (end 169.26 121.69) (width 0.5) (layer "F.Cu") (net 2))
 (segment (start 191.325 125.97) (end 189.22 125.97) (width 0.6) (layer "F.Cu") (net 2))
 (segment (start 116.49 121.69) (end 114.28 121.69) (width 0.5) (layer "F.Cu") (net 2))
 (segment (start 131.56 124.64) (end 134.51 121.69) (width 0.5) (layer "F.Cu") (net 2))
 (segment (start 213.78 120.6) (end 216.33 123.15) (width 0.5) (layer "F.Cu") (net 2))
 (segment (start 171.5 121.69) (end 172.94 121.69) (width 0.5) (layer "F.Cu") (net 2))
 (segment (start 151.71 121.69) (end 147.91 121.69) (width 0.5) (layer "F.Cu") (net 2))
 (segment (start 172.94 121.69) (end 178.11 121.69) (width 0.5) (layer "F.Cu") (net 2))
 (segment (start 154.06 121.69) (end 151.71 121.69) (width 0.5) (layer "F.Cu") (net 2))
 (segment (start 112.22 121.7) (end 106 121.7) (width 0.5) (layer "F.Cu") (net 2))
 (segment (start 171.5 121.69) (end 170.81 121.69) (width 0.5) (layer "F.Cu") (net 2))
 (segment (start 134.51 121.69) (end 126.21 121.69) (width 0.5) (layer "F.Cu") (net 2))
 (segment (start 121.21 121.69) (end 116.49 121.69) (width 0.5) (layer "F.Cu") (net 2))
 (segment (start 126.21 121.69) (end 121.21 121.69) (width 0.5) (layer "F.Cu") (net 2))
 (segment (start 156.57 121.69) (end 154.06 121.69) (width 0.5) (layer "F.Cu") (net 2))
 (segment (start 147.91 121.69) (end 145.71 121.69) (width 0.5) (layer "F.Cu") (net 2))
 (segment (start 173.82 124.7) (end 170.81 121.69) (width 0.5) (layer "F.Cu") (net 2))
 (via (at 175.39 121.7) (size 0.8) (drill 0.4) (layers "F.Cu" "B.Cu") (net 2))
 (via (at 112.22 121.7) (size 0.8) (drill 0.4) (layers "F.Cu" "B.Cu") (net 2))
 (via (at 156.57 121.69) (size 0.8) (drill 0.4) (layers "F.Cu" "B.Cu") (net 2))
 (via (at 145.71 121.69) (size 0.8) (drill 0.4) (layers "F.Cu" "B.Cu") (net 2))
 (via (at 200.1 120.6) (size 0.8) (drill 0.4) (layers "F.Cu" "B.Cu") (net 2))
 (via (at 143.93 121.69) (size 0.8) (drill 0.4) (layers "F.Cu" "B.Cu") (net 2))
 (via (at 178.13 121.7) (size 0.8) (drill 0.4) (layers "F.Cu" "B.Cu") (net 2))
 (via (at 139.5 121.69) (size 0.8) (drill 0.4) (layers "F.Cu" "B.Cu") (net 2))
 (via (at 172.94 121.69) (size 0.8) (drill 0.4) (layers "F.Cu" "B.Cu") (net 2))
 (via (at 114.28 121.69) (size 0.8) (drill 0.4) (layers "F.Cu" "B.Cu") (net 2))
 (via (at 151.71 121.69) (size 0.8) (drill 0.4) (layers "F.Cu" "B.Cu") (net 2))
 (via (at 137.29 121.69) (size 0.8) (drill 0.4) (layers "F.Cu" "B.Cu") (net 2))
 (via (at 184.91 121.7) (size 0.8) (drill 0.4) (layers "F.Cu" "B.Cu") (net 2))
 (via (at 185.79 122.54) (size 0.8) (drill 0.4) (layers "F.Cu" "B.Cu") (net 2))
 (via (at 116.49 121.69) (size 0.8) (drill 0.4) (layers "F.Cu" "B.Cu") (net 2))
 (via (at 154.06 121.69) (size 0.8) (drill 0.4) (layers "F.Cu" "B.Cu") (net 2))
 (segment (start 161.8 121.7) (end 162.1 121.7) (width 0.5) (layer "B.Cu") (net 2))
 (segment (start 101 120.7) (end 88.05 120.7) (width 0.5) (layer "B.Cu") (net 2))
 (segment (start 125.05 124.7) (end 125.05 124.65) (width 0.5) (layer "B.Cu") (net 2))
 (segment (start 200.1 120.6) (end 196.8 120.6) (width 0.5) (layer "B.Cu") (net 2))
 (segment (start 184.28 120.6) (end 183.18 121.7) (width 0.5) (layer "B.Cu") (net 2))
 (segment (start 178.13 121.7) (end 177.64 121.7) (width 0.25) (layer "B.Cu") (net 2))
 (segment (start 192.7 124.7) (end 196.8 120.6) (width 0.5) (layer "B.Cu") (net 2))
 (segment (start 128 121.7) (end 112.22 121.7) (width 0.5) (layer "B.Cu") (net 2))
 (segment (start 185.79 122.54) (end 184.95 121.7) (width 0.5) (layer "B.Cu") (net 2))
 (segment (start 183.18 121.7) (end 178.13 121.7) (width 0.5) (layer "B.Cu") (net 2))
 (segment (start 174.84 121.7) (end 175.39 121.7) (width 0.5) (layer "B.Cu") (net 2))
 (segment (start 192.55 124.7) (end 192.7 124.7) (width 0.5) (layer "B.Cu") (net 2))
 (segment (start 176.25 121.7) (end 177.64 121.7) (width 0.5) (layer "B.Cu") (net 2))
 (segment (start 102 121.7) (end 101 120.7) (width 0.5) (layer "B.Cu") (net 2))
 (segment (start 175.39 121.7) (end 176.25 121.7) (width 0.5) (layer "B.Cu") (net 2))
 (segment (start 184.91 121.7) (end 183.18 121.7) (width 0.5) (layer "B.Cu") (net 2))
 (segment (start 204.55 120.6) (end 204.85 120.9) (width 0.5) (layer "B.Cu") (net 2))
 (segment (start 196.8 120.6) (end 184.28 120.6) (width 0.5) (layer "B.Cu") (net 2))
 (segment (start 158.7875 121.7) (end 134.4 121.7) (width 0.5) (layer "B.Cu") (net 2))
 (segment (start 184.95 121.7) (end 184.91 121.7) (width 0.25) (layer "B.Cu") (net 2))
 (segment (start 200.1 120.6) (end 204.55 120.6) (width 0.5) (layer "B.Cu") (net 2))
 (segment (start 134.4 121.7) (end 128 121.7) (width 0.5) (layer "B.Cu") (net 2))
 (segment (start 112.22 121.7) (end 102 121.7) (width 0.5) (layer "B.Cu") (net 2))
 (segment (start 125.05 124.65) (end 128 121.7) (width 0.5) (layer "B.Cu") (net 2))
 (segment (start 174.84 121.7) (end 162.1 121.7) (width 0.5) (layer "B.Cu") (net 2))
 (segment (start 162.1 121.7) (end 158.7875 121.7) (width 0.5) (layer "B.Cu") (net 2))
 (segment (start 158.8 124.7) (end 161.8 121.7) (width 0.5) (layer "B.Cu") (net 2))
 (segment (start 194.795 128.65) (end 89.45 128.65) (width 0.5) (layer "F.Cu") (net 3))
 (segment (start 89.45 128.65) (end 87.2 126.4) (width 0.5) (layer "F.Cu") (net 3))
 (segment (start 87.2 126.4) (end 87.2 124.7) (width 0.5) (layer "F.Cu") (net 3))
 (segment (start 197.475 125.97) (end 194.795 128.65) (width 0.5) (layer "F.Cu") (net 3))
 (segment (start 204.53 123.43) (end 205.8 124.7) (width 0.2) (layer "F.Cu") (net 4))
 (segment (start 197.475 123.43) (end 204.53 123.43) (width 0.5) (layer "F.Cu") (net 4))
 (segment (start 178.725 124.7) (end 170.05 124.7) (width 0.25) (layer "B.Cu") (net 10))
 (segment (start 164.33 124.7) (end 161.08 127.95) (width 0.25) (layer "B.Cu") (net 11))
 (segment (start 167.475 124.7) (end 164.33 124.7) (width 0.25) (layer "B.Cu") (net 11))
 (segment (start 189.975 124.7) (end 181.3 124.7) (width 0.25) (layer "B.Cu") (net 12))
 (segment (start 156.225 124.7) (end 147.55 124.7) (width 0.25) (layer "B.Cu") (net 14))
 (segment (start 111.225 124.7) (end 102.55 124.7) (width 0.25) (layer "B.Cu") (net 17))
 (segment (start 122.475 124.7) (end 113.8 124.7) (width 0.25) (layer "B.Cu") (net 20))
 (segment (start 99.975 124.7) (end 99.975 126.075) (width 0.25) (layer "B.Cu") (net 18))
 (segment (start 99.975 126.075) (end 101.84 127.94) (width 0.25) (layer "B.Cu") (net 18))
 (segment (start 101.84 127.94) (end 111.75 127.94) (width 0.25) (layer "B.Cu") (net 18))
 (segment (start 71.7 122) (end 71.7 123.65) (width 0.25) (layer "B.Cu") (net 9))
 (segment (start 73 120.7) (end 71.7 122) (width 0.25) (layer "B.Cu") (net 9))
 (segment (start 85.475 120.7) (end 73 120.7) (width 0.25) (layer "B.Cu") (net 9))
 (segment (start 85.95 128.7) (end 73 128.7) (width 0.25) (layer "B.Cu") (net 22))
 (segment (start 71.7 127.4) (end 71.7 126.225) (width 0.25) (layer "B.Cu") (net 22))
 (segment (start 73 128.7) (end 71.7 127.4) (width 0.25) (layer "B.Cu") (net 22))
 (segment (start 93.95 127.94) (end 93.19 128.7) (width 0.25) (layer "B.Cu") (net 13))
 (segment (start 93.19 128.7) (end 88.525 128.7) (width 0.25) (layer "B.Cu") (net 13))
 (segment (start 144.975 124.7) (end 136.3 124.7) (width 0.25) (layer "B.Cu") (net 21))
 (segment (start 143.74 127.94) (end 136.54 127.94) (width 0.25) (layer "B.Cu") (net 8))
 (segment (start 133.725 125.125) (end 133.725 124.7) (width 0.25) (layer "B.Cu") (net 8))
 (segment (start 136.54 127.94) (end 133.725 125.125) (width 0.25) (layer "B.Cu") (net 8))
 (segment (start 207.425 120.9) (end 218.35 120.9) (width 0.25) (layer "B.Cu") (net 19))
 (segment (start 218.35 120.9) (end 221.1 123.65) (width 0.25) (layer "B.Cu") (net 19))
 (segment (start 221.1 127.2) (end 219.6 128.7) (width 0.25) (layer "B.Cu") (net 15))
 (segment (start 219.6 128.7) (end 206.95 128.7) (width 0.25) (layer "B.Cu") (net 15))
 (segment (start 221.1 126.225) (end 221.1 127.2) (width 0.25) (layer "B.Cu") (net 15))
 (segment (start 198 127.7) (end 199 128.7) (width 0.25) (layer "B.Cu") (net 16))
 (segment (start 199 128.7) (end 204.375 128.7) (width 0.25) (layer "B.Cu") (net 16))
 (segment (start 188.16 126.63) (end 192.33 126.63) (width 0.25) (layer "B.Cu") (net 16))
 (segment (start 192.33 126.63) (end 193.4 127.7) (width 0.25) (layer "B.Cu") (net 16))
 (segment (start 193.4 127.7) (end 198 127.7) (width 0.25) (layer "B.Cu") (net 16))
 (segment (start 186.85 127.94) (end 188.16 126.63) (width 0.25) (layer "B.Cu") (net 16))
 (segment (start 216.75 126.25) (end 216.33 126.25) (width 0.25) (layer "F.Cu") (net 7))
 (segment (start 220.64 122.36) (end 216.75 126.25) (width 0.25) (layer "F.Cu") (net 7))
 (segment (start 188.53 123.43) (end 185.8 120.7) (width 0.6) (layer "F.Cu") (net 1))
 (segment (start 184.05 120.7) (end 181.05 123.7) (width 0.6) (layer "F.Cu") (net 1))
 (segment (start 191.325 123.43) (end 188.53 123.43) (width 0.6) (layer "F.Cu") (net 1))
 (segment (start 185.8 120.7) (end 184.05 120.7) (width 0.6) (layer "F.Cu") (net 1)))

